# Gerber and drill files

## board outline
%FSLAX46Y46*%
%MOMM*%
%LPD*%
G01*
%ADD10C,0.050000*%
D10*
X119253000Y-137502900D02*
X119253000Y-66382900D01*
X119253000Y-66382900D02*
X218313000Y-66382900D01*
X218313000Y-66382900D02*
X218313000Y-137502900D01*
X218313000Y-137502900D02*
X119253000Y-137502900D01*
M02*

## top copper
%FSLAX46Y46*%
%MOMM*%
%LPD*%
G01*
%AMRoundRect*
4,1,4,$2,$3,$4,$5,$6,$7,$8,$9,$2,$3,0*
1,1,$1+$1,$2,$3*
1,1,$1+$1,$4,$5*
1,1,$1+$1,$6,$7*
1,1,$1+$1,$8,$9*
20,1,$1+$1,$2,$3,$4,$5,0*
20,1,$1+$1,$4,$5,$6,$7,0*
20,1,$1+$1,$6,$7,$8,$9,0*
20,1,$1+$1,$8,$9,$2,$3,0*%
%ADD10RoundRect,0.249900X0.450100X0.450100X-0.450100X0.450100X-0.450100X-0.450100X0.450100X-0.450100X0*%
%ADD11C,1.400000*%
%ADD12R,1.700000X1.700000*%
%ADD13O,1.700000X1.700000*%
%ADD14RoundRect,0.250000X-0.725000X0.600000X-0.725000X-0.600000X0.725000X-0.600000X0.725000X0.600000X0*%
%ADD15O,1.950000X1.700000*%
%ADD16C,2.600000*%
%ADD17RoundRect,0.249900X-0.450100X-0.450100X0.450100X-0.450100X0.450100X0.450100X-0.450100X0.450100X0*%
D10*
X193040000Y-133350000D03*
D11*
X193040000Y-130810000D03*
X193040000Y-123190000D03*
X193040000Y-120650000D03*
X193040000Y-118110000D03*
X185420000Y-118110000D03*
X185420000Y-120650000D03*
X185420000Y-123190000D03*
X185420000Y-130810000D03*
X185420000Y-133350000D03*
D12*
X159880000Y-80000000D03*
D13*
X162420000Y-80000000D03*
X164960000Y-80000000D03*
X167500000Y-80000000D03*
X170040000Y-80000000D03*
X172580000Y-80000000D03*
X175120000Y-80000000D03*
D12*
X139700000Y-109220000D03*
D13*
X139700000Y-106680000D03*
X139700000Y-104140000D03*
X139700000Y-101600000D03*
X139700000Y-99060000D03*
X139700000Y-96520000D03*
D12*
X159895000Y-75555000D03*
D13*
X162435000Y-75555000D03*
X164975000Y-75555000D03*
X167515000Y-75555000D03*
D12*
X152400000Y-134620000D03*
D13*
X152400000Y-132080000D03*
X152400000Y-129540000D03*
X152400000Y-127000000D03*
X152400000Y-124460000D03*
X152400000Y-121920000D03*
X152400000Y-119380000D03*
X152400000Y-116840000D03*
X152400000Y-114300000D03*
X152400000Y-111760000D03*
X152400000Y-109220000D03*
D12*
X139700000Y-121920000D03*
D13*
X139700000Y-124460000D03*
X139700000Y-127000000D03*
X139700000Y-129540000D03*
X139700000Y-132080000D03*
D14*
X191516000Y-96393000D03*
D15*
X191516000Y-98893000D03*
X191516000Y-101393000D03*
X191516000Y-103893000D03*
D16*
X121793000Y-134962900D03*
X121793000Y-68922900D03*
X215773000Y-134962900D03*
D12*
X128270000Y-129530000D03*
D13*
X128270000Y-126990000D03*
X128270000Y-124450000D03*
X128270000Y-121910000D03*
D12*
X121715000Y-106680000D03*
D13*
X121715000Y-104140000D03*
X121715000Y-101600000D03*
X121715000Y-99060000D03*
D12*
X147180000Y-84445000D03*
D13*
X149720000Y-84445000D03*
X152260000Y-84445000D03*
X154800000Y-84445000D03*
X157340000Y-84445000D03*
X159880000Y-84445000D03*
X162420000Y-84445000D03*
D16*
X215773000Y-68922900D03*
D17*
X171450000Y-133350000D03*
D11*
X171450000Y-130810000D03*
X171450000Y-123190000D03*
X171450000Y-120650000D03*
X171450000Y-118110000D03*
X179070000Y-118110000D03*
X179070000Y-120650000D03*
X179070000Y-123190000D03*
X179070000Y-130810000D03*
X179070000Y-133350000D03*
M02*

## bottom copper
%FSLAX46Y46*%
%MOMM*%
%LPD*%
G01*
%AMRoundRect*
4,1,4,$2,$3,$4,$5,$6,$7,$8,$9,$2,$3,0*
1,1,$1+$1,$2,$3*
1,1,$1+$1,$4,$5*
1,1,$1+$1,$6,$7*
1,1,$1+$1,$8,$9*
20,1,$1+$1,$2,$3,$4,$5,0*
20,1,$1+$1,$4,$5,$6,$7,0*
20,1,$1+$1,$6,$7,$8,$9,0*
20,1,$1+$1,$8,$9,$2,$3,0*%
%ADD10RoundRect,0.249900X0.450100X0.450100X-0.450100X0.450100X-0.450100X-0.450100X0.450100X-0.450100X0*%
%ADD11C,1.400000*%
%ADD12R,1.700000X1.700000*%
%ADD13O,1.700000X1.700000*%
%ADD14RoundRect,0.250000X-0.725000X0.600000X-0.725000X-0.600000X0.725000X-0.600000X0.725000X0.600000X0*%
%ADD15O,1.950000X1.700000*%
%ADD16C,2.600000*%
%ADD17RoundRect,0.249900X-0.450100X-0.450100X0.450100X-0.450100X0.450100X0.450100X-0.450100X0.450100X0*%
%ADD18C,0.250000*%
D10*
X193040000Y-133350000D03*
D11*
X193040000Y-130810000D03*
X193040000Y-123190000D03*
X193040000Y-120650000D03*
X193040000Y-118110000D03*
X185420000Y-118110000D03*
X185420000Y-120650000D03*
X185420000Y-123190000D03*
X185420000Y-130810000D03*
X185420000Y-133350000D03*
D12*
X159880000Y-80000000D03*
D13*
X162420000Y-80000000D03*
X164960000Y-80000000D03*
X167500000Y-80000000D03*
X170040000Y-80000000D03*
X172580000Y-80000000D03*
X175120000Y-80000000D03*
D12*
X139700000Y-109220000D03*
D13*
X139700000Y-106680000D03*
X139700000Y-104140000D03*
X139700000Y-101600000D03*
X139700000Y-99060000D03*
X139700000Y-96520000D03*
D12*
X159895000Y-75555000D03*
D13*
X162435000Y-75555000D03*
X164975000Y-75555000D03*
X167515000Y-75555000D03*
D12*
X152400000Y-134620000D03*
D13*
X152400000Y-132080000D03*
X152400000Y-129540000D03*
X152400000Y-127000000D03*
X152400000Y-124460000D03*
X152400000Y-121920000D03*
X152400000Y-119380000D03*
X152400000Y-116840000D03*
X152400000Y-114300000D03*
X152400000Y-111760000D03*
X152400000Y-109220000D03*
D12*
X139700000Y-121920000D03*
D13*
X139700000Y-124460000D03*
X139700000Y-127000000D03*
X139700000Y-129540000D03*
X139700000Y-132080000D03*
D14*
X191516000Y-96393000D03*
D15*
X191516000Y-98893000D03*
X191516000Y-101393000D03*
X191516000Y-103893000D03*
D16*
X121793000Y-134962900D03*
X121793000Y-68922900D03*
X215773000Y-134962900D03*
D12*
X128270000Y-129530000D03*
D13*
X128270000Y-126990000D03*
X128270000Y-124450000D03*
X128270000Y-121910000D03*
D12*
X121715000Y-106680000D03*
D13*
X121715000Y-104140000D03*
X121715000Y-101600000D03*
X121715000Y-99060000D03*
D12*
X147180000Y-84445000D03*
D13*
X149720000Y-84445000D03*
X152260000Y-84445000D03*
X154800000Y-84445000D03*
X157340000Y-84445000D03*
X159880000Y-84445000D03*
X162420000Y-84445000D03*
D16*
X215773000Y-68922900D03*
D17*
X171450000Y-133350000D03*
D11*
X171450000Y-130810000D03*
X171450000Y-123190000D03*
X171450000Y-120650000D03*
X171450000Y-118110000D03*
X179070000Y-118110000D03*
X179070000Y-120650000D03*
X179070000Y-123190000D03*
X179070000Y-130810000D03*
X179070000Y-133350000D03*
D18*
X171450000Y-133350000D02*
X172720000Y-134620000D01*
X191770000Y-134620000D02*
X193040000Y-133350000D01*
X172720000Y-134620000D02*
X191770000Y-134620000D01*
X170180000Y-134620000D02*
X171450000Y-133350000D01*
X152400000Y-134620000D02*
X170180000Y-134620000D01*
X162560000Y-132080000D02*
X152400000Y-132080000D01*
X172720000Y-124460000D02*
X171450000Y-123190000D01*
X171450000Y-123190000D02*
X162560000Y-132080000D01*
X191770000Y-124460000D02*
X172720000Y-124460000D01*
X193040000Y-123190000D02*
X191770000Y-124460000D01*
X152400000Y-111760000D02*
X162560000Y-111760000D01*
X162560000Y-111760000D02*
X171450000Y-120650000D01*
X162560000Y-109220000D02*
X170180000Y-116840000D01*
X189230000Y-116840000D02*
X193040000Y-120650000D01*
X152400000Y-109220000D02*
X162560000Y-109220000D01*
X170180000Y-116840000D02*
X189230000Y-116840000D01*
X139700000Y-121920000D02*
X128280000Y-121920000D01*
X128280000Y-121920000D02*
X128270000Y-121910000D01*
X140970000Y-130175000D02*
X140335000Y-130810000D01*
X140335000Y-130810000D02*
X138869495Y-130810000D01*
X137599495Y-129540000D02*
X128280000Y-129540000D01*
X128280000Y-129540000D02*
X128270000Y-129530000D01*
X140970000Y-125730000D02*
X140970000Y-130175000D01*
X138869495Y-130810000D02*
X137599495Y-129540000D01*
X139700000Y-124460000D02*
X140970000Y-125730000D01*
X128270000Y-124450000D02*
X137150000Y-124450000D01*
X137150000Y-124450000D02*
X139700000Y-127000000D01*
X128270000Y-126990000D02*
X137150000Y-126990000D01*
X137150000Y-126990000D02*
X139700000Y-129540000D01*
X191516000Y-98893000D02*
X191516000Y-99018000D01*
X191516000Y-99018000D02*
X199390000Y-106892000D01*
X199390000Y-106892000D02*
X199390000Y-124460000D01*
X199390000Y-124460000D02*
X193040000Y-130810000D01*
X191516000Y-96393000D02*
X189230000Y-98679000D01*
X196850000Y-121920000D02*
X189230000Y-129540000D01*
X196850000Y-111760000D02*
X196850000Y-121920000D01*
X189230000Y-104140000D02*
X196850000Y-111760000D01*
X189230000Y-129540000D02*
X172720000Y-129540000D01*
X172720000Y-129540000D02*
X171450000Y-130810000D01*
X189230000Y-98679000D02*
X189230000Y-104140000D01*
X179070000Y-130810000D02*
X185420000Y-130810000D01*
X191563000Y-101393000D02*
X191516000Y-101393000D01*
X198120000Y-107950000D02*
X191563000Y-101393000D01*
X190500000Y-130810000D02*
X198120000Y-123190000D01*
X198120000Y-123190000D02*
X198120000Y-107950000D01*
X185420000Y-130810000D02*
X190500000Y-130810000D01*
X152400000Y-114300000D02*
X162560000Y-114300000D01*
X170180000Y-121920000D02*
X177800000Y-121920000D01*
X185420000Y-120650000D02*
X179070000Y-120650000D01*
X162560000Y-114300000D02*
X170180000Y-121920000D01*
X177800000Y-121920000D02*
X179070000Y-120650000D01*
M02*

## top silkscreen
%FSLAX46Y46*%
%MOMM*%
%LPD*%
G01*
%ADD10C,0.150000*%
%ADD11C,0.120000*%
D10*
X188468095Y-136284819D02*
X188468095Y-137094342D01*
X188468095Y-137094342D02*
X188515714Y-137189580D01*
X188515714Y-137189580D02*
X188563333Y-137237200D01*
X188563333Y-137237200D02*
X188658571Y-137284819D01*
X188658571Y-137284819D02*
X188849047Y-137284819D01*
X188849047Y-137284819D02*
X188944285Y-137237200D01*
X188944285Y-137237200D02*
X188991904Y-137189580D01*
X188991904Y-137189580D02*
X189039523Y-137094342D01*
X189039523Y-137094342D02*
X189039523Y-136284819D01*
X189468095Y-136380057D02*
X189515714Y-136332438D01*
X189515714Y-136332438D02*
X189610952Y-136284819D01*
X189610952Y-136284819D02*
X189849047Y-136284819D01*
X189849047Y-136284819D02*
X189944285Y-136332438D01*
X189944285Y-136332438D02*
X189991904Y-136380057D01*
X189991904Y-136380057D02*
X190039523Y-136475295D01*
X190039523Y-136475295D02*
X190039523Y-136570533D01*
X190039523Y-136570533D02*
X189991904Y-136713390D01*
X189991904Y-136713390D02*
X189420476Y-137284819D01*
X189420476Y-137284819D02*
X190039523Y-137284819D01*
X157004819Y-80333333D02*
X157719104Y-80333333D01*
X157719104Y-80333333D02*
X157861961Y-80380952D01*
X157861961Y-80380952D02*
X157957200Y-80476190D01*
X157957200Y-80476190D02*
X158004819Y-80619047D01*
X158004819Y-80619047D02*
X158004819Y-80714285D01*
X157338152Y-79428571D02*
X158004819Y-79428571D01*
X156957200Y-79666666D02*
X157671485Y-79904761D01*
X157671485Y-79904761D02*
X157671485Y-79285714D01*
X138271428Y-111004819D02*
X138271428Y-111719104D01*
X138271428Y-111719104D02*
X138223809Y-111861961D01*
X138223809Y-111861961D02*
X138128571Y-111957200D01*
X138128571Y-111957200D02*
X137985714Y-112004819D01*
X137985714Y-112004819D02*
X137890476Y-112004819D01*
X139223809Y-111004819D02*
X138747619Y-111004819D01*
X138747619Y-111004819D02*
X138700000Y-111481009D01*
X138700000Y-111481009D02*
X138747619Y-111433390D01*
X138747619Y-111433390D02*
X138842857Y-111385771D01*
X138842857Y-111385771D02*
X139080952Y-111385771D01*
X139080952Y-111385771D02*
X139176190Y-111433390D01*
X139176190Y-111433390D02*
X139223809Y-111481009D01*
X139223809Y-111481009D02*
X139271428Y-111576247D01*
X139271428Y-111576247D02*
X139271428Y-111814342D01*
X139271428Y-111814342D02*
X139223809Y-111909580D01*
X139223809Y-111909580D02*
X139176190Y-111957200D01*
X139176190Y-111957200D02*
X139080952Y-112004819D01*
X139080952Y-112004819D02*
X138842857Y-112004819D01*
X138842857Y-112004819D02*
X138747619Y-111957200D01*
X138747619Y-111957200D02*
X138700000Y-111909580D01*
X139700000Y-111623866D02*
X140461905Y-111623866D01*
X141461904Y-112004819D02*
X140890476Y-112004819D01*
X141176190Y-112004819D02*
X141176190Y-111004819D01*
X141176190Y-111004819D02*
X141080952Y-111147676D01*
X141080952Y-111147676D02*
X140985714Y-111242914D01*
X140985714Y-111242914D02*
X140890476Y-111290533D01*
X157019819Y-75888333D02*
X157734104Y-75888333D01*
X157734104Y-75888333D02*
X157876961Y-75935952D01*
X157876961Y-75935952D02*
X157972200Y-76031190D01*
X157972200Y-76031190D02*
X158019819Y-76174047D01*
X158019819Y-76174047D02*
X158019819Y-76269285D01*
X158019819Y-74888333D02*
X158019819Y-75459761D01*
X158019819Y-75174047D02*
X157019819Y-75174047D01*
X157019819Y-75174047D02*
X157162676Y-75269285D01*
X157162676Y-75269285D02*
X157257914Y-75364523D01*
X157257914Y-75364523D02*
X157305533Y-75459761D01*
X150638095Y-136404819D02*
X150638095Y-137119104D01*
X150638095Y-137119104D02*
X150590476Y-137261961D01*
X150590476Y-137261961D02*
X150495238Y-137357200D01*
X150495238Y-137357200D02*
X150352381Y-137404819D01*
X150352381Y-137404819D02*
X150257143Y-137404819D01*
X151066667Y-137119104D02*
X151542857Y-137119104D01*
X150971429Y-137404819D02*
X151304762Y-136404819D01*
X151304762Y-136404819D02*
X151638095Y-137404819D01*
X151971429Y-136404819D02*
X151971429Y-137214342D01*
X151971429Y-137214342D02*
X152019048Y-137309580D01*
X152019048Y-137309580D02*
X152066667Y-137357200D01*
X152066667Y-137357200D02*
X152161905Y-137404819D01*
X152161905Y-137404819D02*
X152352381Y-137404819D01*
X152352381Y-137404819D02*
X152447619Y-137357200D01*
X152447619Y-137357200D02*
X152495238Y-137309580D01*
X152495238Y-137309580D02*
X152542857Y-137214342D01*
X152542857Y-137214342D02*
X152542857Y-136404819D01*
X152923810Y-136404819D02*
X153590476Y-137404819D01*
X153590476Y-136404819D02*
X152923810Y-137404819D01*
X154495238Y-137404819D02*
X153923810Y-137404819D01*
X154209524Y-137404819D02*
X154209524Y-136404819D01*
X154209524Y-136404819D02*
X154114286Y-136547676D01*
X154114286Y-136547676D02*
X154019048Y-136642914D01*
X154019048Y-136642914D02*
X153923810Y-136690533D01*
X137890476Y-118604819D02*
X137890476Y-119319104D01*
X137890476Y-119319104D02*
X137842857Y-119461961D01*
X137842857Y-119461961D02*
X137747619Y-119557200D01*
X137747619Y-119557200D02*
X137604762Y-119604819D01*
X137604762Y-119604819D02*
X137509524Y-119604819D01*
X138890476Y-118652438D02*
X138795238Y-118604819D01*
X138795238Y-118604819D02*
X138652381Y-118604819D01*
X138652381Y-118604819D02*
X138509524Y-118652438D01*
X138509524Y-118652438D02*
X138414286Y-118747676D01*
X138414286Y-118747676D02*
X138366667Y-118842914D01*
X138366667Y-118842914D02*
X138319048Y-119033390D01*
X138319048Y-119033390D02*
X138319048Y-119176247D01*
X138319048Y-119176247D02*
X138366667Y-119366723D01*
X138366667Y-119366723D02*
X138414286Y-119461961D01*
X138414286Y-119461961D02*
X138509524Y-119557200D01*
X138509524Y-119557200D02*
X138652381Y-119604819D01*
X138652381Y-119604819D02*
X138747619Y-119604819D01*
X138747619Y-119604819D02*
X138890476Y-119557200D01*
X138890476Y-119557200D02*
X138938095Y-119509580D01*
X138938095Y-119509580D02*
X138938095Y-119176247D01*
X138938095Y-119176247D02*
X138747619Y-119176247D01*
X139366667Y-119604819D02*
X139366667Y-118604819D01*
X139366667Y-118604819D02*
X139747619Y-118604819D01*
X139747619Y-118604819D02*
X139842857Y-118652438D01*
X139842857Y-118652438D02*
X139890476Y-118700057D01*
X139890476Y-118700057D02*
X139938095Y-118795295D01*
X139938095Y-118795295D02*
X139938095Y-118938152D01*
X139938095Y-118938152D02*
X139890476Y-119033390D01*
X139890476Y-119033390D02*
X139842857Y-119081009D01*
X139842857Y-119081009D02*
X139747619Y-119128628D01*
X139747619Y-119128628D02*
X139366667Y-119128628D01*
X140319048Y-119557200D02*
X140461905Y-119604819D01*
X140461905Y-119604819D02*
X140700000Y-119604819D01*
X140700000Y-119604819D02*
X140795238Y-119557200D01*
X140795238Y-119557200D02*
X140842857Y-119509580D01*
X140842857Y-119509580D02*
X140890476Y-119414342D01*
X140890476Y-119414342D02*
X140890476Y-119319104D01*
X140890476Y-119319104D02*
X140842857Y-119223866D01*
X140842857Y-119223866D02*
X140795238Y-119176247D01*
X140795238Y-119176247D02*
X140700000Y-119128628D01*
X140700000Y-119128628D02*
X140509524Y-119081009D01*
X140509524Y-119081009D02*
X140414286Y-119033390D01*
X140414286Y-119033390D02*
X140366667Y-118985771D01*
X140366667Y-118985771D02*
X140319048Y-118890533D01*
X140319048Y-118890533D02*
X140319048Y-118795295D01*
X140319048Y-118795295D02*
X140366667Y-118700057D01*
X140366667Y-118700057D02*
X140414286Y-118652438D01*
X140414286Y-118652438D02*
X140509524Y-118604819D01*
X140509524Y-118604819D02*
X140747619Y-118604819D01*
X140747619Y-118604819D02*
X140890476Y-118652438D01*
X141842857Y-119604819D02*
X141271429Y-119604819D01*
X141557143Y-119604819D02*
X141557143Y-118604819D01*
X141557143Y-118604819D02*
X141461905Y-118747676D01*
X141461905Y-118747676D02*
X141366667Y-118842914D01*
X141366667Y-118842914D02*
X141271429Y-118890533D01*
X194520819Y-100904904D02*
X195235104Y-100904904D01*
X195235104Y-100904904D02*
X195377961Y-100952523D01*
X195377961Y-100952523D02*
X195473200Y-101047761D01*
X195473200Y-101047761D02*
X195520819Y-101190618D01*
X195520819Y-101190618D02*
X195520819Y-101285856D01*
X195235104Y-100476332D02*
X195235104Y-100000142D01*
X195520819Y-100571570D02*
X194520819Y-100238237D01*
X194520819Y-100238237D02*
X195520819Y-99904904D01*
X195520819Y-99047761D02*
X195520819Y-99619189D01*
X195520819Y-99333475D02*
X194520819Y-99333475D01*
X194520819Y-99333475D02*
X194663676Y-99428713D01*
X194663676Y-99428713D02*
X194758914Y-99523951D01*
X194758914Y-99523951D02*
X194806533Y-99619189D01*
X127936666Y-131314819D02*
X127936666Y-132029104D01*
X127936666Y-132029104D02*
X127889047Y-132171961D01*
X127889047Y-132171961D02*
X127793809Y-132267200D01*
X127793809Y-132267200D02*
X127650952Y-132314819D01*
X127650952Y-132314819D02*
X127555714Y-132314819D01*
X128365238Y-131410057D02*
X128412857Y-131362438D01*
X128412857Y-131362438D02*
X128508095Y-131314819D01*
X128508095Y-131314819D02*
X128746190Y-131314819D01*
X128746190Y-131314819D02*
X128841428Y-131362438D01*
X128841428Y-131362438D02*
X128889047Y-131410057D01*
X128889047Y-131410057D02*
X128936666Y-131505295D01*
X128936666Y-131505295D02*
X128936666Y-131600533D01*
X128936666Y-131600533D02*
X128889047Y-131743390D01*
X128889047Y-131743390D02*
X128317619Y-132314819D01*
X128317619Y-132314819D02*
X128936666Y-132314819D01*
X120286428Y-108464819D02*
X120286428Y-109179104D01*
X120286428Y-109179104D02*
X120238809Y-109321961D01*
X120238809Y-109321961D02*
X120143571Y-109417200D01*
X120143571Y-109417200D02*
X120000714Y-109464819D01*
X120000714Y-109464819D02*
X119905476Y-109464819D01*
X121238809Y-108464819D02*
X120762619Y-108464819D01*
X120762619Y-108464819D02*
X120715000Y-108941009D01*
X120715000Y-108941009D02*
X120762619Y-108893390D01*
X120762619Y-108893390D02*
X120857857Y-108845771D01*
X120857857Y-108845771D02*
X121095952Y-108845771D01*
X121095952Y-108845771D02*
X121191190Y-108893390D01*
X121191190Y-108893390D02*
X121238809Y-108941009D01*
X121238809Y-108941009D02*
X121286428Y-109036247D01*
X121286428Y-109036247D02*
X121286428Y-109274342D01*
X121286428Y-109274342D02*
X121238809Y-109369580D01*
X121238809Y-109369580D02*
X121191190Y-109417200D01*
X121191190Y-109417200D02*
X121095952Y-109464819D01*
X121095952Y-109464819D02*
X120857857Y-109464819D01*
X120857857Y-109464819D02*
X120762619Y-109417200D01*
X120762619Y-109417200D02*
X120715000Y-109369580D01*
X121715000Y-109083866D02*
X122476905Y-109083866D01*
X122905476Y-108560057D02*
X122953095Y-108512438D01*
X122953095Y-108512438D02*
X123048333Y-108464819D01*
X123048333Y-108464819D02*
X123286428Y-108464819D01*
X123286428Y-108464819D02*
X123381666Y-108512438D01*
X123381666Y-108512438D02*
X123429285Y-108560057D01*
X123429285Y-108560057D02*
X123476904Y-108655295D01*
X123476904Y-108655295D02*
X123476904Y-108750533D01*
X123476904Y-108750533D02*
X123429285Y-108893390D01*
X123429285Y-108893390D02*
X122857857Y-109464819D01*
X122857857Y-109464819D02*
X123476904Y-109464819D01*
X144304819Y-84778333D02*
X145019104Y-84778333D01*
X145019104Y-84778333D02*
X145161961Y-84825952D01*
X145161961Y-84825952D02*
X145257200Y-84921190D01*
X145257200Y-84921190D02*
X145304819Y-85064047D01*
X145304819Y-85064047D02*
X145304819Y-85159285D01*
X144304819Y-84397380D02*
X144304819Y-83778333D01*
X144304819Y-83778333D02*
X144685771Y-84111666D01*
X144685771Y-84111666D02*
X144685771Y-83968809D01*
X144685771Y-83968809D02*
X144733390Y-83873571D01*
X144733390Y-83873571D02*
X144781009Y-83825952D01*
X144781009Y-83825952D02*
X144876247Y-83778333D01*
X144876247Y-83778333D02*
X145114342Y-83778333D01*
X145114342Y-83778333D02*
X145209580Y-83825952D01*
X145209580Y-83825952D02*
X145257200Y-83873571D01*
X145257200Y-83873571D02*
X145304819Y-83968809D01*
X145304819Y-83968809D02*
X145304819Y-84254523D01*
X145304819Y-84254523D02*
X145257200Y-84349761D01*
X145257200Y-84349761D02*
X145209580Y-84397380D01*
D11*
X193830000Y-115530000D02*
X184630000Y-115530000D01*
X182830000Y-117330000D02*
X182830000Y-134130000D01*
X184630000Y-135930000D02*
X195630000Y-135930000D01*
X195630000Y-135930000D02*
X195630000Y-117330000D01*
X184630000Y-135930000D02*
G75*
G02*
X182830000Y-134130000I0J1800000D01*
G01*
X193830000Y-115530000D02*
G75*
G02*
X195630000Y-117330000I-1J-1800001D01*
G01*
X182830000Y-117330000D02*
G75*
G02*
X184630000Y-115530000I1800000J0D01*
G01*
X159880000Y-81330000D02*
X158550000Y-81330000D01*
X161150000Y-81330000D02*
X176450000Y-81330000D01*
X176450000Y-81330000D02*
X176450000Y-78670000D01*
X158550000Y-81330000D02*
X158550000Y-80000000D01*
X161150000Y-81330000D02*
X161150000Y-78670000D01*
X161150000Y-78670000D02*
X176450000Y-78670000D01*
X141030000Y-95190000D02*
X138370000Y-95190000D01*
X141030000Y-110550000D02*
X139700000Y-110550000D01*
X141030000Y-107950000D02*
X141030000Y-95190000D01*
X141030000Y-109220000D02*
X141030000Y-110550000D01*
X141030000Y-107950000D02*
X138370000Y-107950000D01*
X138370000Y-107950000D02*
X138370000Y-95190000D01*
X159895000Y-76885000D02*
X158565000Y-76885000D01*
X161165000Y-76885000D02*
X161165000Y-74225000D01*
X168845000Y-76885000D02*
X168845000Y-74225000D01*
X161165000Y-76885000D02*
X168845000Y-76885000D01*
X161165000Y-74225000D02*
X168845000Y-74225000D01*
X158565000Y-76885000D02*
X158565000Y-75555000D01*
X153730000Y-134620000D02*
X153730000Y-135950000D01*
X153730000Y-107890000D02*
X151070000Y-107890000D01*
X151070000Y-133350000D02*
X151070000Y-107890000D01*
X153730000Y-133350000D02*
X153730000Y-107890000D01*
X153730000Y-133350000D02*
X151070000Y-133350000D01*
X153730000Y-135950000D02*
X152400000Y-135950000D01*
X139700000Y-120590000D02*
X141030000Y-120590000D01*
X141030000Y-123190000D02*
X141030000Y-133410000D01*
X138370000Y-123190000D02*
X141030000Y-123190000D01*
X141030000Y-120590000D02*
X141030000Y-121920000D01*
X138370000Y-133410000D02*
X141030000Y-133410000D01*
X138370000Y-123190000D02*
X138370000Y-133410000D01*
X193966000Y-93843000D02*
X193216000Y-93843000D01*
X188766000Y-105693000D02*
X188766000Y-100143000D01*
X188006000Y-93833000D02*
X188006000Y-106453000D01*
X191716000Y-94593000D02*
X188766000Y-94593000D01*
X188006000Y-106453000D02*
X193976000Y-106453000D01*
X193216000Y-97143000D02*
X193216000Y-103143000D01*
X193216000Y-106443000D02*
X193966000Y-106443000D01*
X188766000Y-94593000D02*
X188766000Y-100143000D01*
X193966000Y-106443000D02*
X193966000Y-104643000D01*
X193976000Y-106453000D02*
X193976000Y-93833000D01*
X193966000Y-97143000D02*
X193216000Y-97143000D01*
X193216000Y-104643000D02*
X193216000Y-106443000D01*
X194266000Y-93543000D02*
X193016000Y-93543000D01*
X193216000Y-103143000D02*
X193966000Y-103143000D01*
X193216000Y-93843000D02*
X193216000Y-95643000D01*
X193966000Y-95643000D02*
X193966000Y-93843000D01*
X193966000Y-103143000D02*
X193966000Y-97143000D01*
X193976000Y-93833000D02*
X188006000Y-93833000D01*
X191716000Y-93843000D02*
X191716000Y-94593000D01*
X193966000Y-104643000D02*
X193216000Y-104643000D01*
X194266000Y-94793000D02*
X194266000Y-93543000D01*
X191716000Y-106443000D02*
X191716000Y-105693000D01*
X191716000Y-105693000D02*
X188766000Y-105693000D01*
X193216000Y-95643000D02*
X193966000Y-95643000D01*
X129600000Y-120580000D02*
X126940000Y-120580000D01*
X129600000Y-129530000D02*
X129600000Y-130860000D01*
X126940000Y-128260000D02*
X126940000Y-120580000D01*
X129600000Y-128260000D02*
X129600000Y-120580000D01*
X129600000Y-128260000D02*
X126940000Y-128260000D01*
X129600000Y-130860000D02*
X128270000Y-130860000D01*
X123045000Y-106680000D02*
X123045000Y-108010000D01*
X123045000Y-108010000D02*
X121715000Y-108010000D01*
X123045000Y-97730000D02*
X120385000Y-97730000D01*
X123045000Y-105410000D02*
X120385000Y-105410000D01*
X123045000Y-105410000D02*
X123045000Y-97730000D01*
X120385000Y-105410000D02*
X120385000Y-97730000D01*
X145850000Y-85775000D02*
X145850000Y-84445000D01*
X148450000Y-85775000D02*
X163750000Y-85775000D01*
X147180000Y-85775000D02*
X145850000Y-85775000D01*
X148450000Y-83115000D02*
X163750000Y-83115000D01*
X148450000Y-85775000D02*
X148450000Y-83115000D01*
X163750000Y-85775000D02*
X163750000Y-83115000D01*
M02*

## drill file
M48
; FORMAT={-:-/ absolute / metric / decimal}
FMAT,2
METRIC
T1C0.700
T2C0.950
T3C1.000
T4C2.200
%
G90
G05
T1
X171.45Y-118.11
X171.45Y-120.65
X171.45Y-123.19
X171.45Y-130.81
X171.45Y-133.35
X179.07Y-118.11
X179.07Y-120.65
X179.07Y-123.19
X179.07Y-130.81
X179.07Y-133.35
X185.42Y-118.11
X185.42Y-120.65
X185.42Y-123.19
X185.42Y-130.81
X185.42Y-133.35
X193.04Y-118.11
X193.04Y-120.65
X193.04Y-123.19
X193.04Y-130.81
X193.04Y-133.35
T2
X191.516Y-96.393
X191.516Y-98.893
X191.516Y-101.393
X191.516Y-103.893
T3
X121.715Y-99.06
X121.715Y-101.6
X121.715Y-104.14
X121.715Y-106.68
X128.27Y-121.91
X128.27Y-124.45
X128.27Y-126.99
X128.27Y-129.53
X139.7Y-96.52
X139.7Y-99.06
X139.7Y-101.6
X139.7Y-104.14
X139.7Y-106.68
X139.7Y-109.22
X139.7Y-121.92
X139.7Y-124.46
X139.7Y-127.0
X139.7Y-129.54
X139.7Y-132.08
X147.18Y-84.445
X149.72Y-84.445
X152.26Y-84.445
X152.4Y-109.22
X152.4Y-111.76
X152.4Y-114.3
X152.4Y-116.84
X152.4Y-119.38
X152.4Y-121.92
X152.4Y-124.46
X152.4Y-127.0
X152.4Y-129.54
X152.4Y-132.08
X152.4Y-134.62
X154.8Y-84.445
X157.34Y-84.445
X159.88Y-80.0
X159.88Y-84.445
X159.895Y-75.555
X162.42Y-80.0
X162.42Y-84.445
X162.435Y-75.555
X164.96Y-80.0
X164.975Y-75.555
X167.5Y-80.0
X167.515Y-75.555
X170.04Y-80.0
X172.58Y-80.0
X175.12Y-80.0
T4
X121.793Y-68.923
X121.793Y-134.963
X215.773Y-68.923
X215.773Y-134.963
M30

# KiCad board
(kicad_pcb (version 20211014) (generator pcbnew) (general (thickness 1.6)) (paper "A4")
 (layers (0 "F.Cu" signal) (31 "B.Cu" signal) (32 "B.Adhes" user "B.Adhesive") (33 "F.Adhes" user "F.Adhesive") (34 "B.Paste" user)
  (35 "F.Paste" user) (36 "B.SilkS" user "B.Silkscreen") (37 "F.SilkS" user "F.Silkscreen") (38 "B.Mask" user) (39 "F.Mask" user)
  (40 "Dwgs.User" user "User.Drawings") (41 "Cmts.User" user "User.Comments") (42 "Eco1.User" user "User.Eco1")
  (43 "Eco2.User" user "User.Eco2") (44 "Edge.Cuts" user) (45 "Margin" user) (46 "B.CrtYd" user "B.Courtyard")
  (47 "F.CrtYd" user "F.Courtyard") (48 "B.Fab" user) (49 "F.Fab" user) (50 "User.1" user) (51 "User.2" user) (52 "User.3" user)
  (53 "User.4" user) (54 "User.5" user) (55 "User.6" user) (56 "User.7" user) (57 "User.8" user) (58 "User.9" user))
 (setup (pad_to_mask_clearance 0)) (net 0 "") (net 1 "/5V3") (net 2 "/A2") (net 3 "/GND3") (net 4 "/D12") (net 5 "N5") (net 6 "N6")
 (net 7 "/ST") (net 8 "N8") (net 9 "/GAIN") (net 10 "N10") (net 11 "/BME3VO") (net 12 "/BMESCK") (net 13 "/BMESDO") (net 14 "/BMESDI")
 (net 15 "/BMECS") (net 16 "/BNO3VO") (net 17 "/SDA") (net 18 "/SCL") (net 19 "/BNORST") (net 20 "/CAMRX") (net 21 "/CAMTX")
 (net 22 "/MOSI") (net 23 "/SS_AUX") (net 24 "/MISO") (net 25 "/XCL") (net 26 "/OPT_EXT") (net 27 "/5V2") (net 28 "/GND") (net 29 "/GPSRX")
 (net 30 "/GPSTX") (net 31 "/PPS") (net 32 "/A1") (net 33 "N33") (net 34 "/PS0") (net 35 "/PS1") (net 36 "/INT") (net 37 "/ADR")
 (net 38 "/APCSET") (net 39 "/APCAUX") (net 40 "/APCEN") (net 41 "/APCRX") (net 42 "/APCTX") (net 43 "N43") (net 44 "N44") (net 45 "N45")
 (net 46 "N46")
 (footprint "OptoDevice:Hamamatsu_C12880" (layer "F.Cu") (at 193.04 133.35 180)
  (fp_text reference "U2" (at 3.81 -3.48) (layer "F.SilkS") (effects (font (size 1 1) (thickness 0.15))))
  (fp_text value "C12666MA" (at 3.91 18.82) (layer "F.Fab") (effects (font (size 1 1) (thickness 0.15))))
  (fp_line (start -0.79 17.82) (end 8.41 17.82) (layer "F.SilkS") (width 0.12))
  (fp_line (start 10.21 16.02) (end 10.21 -0.78) (layer "F.SilkS") (width 0.12))
  (fp_line (start 8.41 -2.58) (end -2.59 -2.58) (layer "F.SilkS") (width 0.12))
  (fp_line (start -2.59 -2.58) (end -2.59 16.02) (layer "F.SilkS") (width 0.12))
  (fp_arc (start 8.41 -2.58) (mid 9.682792 -2.052792) (end 10.21 -0.78) (layer "F.SilkS") (width 0.12))
  (fp_arc (start -0.79 17.82) (mid -2.062792 17.292792) (end -2.59 16.02) (layer "F.SilkS") (width 0.12))
  (fp_arc (start 10.21 16.02) (mid 9.682792 17.292792) (end 8.41 17.82) (layer "F.SilkS") (width 0.12))
  (pad "1" thru_hole roundrect (at 0 0 180) (size 1.4 1.4) (drill 0.7) (layers *.Cu *.Mask) (roundrect_rratio 0.1785) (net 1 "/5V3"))
  (pad "2" thru_hole circle (at 0 2.54 180) (size 1.4 1.4) (drill 0.7) (layers *.Cu *.Mask) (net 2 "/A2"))
  (pad "3" thru_hole circle (at 0 10.16 180) (size 1.4 1.4) (drill 0.7) (layers *.Cu *.Mask) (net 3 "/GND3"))
  (pad "4" thru_hole circle (at 0 12.7 180) (size 1.4 1.4) (drill 0.7) (layers *.Cu *.Mask) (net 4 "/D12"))
  (pad "5" thru_hole circle (at 0 15.24 180) (size 1.4 1.4) (drill 0.7) (layers *.Cu *.Mask) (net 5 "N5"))
  (pad "6" thru_hole circle (at 7.62 15.24 180) (size 1.4 1.4) (drill 0.7) (layers *.Cu *.Mask) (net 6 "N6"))
  (pad "7" thru_hole circle (at 7.62 12.7 180) (size 1.4 1.4) (drill 0.7) (layers *.Cu *.Mask) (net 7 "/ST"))
  (pad "8" thru_hole circle (at 7.62 10.16 180) (size 1.4 1.4) (drill 0.7) (layers *.Cu *.Mask) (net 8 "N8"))
  (pad "9" thru_hole circle (at 7.62 2.54 180) (size 1.4 1.4) (drill 0.7) (layers *.Cu *.Mask) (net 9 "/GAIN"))
  (pad "10" thru_hole circle (at 7.62 0 180) (size 1.4 1.4) (drill 0.7) (layers *.Cu *.Mask) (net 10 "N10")))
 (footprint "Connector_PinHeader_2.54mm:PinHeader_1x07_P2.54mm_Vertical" (layer "F.Cu") (at 159.88 80 90)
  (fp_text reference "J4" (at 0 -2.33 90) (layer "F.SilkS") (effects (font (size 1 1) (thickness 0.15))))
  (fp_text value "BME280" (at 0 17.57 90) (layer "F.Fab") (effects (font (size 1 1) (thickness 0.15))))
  (fp_line (start -1.33 0) (end -1.33 -1.33) (layer "F.SilkS") (width 0.12))
  (fp_line (start -1.33 1.27) (end -1.33 16.57) (layer "F.SilkS") (width 0.12))
  (fp_line (start -1.33 16.57) (end 1.33 16.57) (layer "F.SilkS") (width 0.12))
  (fp_line (start -1.33 -1.33) (end 0 -1.33) (layer "F.SilkS") (width 0.12))
  (fp_line (start -1.33 1.27) (end 1.33 1.27) (layer "F.SilkS") (width 0.12))
  (fp_line (start 1.33 1.27) (end 1.33 16.57) (layer "F.SilkS") (width 0.12))
  (pad "1" thru_hole rect (at 0 0 90) (size 1.7 1.7) (drill 1) (layers *.Cu *.Mask) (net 1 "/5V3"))
  (pad "2" thru_hole oval (at 0 2.54 90) (size 1.7 1.7) (drill 1) (layers *.Cu *.Mask) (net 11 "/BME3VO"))
  (pad "3" thru_hole oval (at 0 5.08 90) (size 1.7 1.7) (drill 1) (layers *.Cu *.Mask) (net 3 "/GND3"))
  (pad "4" thru_hole oval (at 0 7.62 90) (size 1.7 1.7) (drill 1) (layers *.Cu *.Mask) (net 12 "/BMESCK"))
  (pad "5" thru_hole oval (at 0 10.16 90) (size 1.7 1.7) (drill 1) (layers *.Cu *.Mask) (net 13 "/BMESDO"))
  (pad "6" thru_hole oval (at 0 12.7 90) (size 1.7 1.7) (drill 1) (layers *.Cu *.Mask) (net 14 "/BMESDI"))
  (pad "7" thru_hole oval (at 0 15.24 90) (size 1.7 1.7) (drill 1) (layers *.Cu *.Mask) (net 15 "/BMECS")))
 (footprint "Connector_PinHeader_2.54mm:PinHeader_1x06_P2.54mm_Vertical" (layer "F.Cu") (at 139.7 109.22 180)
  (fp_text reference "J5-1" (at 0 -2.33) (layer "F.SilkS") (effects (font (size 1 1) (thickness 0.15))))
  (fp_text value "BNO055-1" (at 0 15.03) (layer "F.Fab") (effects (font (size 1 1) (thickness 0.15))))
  (fp_line (start -1.33 14.03) (end 1.33 14.03) (layer "F.SilkS") (width 0.12))
  (fp_line (start -1.33 -1.33) (end 0 -1.33) (layer "F.SilkS") (width 0.12))
  (fp_line (start -1.33 1.27) (end -1.33 14.03) (layer "F.SilkS") (width 0.12))
  (fp_line (start -1.33 0) (end -1.33 -1.33) (layer "F.SilkS") (width 0.12))
  (fp_line (start -1.33 1.27) (end 1.33 1.27) (layer "F.SilkS") (width 0.12))
  (fp_line (start 1.33 1.27) (end 1.33 14.03) (layer "F.SilkS") (width 0.12))
  (pad "1" thru_hole rect (at 0 0 180) (size 1.7 1.7) (drill 1) (layers *.Cu *.Mask) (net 1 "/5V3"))
  (pad "2" thru_hole oval (at 0 2.54 180) (size 1.7 1.7) (drill 1) (layers *.Cu *.Mask) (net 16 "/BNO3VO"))
  (pad "3" thru_hole oval (at 0 5.08 180) (size 1.7 1.7) (drill 1) (layers *.Cu *.Mask) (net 3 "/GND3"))
  (pad "4" thru_hole oval (at 0 7.62 180) (size 1.7 1.7) (drill 1) (layers *.Cu *.Mask) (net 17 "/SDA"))
  (pad "5" thru_hole oval (at 0 10.16 180) (size 1.7 1.7) (drill 1) (layers *.Cu *.Mask) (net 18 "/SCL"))
  (pad "6" thru_hole oval (at 0 12.7 180) (size 1.7 1.7) (drill 1) (layers *.Cu *.Mask) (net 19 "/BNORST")))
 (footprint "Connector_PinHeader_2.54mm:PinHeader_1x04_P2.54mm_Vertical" (layer "F.Cu") (at 159.895 75.555 90)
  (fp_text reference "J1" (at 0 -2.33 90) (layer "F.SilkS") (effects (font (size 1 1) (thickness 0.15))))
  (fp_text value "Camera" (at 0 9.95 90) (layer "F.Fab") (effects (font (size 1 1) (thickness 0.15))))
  (fp_line (start -1.33 0) (end -1.33 -1.33) (layer "F.SilkS") (width 0.12))
  (fp_line (start -1.33 1.27) (end 1.33 1.27) (layer "F.SilkS") (width 0.12))
  (fp_line (start -1.33 8.95) (end 1.33 8.95) (layer "F.SilkS") (width 0.12))
  (fp_line (start -1.33 1.27) (end -1.33 8.95) (layer "F.SilkS") (width 0.12))
  (fp_line (start 1.33 1.27) (end 1.33 8.95) (layer "F.SilkS") (width 0.12))
  (fp_line (start -1.33 -1.33) (end 0 -1.33) (layer "F.SilkS") (width 0.12))
  (pad "1" thru_hole rect (at 0 0 90) (size 1.7 1.7) (drill 1) (layers *.Cu *.Mask) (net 1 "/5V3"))
  (pad "2" thru_hole oval (at 0 2.54 90) (size 1.7 1.7) (drill 1) (layers *.Cu *.Mask) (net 3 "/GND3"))
  (pad "3" thru_hole oval (at 0 5.08 90) (size 1.7 1.7) (drill 1) (layers *.Cu *.Mask) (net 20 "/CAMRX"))
  (pad "4" thru_hole oval (at 0 7.62 90) (size 1.7 1.7) (drill 1) (layers *.Cu *.Mask) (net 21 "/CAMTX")))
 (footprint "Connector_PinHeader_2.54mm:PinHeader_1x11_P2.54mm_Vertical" (layer "F.Cu") (at 152.4 134.62 180)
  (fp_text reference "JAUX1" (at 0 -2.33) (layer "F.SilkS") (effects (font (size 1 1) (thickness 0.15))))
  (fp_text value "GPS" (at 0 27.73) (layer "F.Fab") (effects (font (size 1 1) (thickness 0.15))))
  (fp_line (start -1.33 0) (end -1.33 -1.33) (layer "F.SilkS") (width 0.12))
  (fp_line (start -1.33 26.73) (end 1.33 26.73) (layer "F.SilkS") (width 0.12))
  (fp_line (start 1.33 1.27) (end 1.33 26.73) (layer "F.SilkS") (width 0.12))
  (fp_line (start -1.33 1.27) (end -1.33 26.73) (layer "F.SilkS") (width 0.12))
  (fp_line (start -1.33 1.27) (end 1.33 1.27) (layer "F.SilkS") (width 0.12))
  (fp_line (start -1.33 -1.33) (end 0 -1.33) (layer "F.SilkS") (width 0.12))
  (pad "1" thru_hole rect (at 0 0 180) (size 1.7 1.7) (drill 1) (layers *.Cu *.Mask) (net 1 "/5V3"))
  (pad "2" thru_hole oval (at 0 2.54 180) (size 1.7 1.7) (drill 1) (layers *.Cu *.Mask) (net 3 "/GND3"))
  (pad "3" thru_hole oval (at 0 5.08 180) (size 1.7 1.7) (drill 1) (layers *.Cu *.Mask) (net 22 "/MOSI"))
  (pad "4" thru_hole oval (at 0 7.62 180) (size 1.7 1.7) (drill 1) (layers *.Cu *.Mask) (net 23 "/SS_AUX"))
  (pad "5" thru_hole oval (at 0 10.16 180) (size 1.7 1.7) (drill 1) (layers *.Cu *.Mask) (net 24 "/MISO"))
  (pad "6" thru_hole oval (at 0 12.7 180) (size 1.7 1.7) (drill 1) (layers *.Cu *.Mask) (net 18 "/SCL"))
  (pad "7" thru_hole oval (at 0 15.24 180) (size 1.7 1.7) (drill 1) (layers *.Cu *.Mask) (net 17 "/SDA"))
  (pad "8" thru_hole oval (at 0 17.78 180) (size 1.7 1.7) (drill 1) (layers *.Cu *.Mask) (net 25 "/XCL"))
  (pad "9" thru_hole oval (at 0 20.32 180) (size 1.7 1.7) (drill 1) (layers *.Cu *.Mask) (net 7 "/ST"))
  (pad "10" thru_hole oval (at 0 22.86 180) (size 1.7 1.7) (drill 1) (layers *.Cu *.Mask) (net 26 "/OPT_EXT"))
  (pad "11" thru_hole oval (at 0 25.4 180) (size 1.7 1.7) (drill 1) (layers *.Cu *.Mask) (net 4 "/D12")))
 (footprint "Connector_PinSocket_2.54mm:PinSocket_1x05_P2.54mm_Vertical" (layer "F.Cu") (at 139.7 121.92)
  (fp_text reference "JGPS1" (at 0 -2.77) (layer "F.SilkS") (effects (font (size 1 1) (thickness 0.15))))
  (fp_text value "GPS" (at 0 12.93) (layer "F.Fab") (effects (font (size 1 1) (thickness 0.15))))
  (fp_line (start 0 -1.33) (end 1.33 -1.33) (layer "F.SilkS") (width 0.12))
  (fp_line (start 1.33 1.27) (end 1.33 11.49) (layer "F.SilkS") (width 0.12))
  (fp_line (start -1.33 1.27) (end 1.33 1.27) (layer "F.SilkS") (width 0.12))
  (fp_line (start 1.33 -1.33) (end 1.33 0) (layer "F.SilkS") (width 0.12))
  (fp_line (start -1.33 11.49) (end 1.33 11.49) (layer "F.SilkS") (width 0.12))
  (fp_line (start -1.33 1.27) (end -1.33 11.49) (layer "F.SilkS") (width 0.12))
  (pad "1" thru_hole rect (at 0 0) (size 1.7 1.7) (drill 1) (layers *.Cu *.Mask) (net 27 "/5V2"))
  (pad "2" thru_hole oval (at 0 2.54) (size 1.7 1.7) (drill 1) (layers *.Cu *.Mask) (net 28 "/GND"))
  (pad "3" thru_hole oval (at 0 5.08) (size 1.7 1.7) (drill 1) (layers *.Cu *.Mask) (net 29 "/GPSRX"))
  (pad "4" thru_hole oval (at 0 7.62) (size 1.7 1.7) (drill 1) (layers *.Cu *.Mask) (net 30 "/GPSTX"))
  (pad "5" thru_hole oval (at 0 10.16) (size 1.7 1.7) (drill 1) (layers *.Cu *.Mask) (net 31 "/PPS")))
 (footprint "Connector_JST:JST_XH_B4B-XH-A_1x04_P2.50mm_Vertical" (layer "F.Cu") (at 191.516 96.393 -90)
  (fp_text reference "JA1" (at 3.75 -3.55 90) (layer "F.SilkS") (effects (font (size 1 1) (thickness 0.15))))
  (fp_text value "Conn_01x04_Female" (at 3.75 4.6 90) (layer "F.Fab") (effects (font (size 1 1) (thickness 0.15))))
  (fp_line (start -2.55 -2.45) (end -2.55 -1.7) (layer "F.SilkS") (width 0.12))
  (fp_line (start 9.3 2.75) (end 3.75 2.75) (layer "F.SilkS") (width 0.12))
  (fp_line (start -2.56 3.51) (end 10.06 3.51) (layer "F.SilkS") (width 0.12))
  (fp_line (start -1.8 -0.2) (end -1.8 2.75) (layer "F.SilkS") (width 0.12))
  (fp_line (start 10.06 3.51) (end 10.06 -2.46) (layer "F.SilkS") (width 0.12))
  (fp_line (start 0.75 -1.7) (end 6.75 -1.7) (layer "F.SilkS") (width 0.12))
  (fp_line (start 10.05 -1.7) (end 10.05 -2.45) (layer "F.SilkS") (width 0.12))
  (fp_line (start -1.8 2.75) (end 3.75 2.75) (layer "F.SilkS") (width 0.12))
  (fp_line (start 10.05 -2.45) (end 8.25 -2.45) (layer "F.SilkS") (width 0.12))
  (fp_line (start 10.06 -2.46) (end -2.56 -2.46) (layer "F.SilkS") (width 0.12))
  (fp_line (start 0.75 -2.45) (end 0.75 -1.7) (layer "F.SilkS") (width 0.12))
  (fp_line (start 8.25 -1.7) (end 10.05 -1.7) (layer "F.SilkS") (width 0.12))
  (fp_line (start -2.85 -2.75) (end -2.85 -1.5) (layer "F.SilkS") (width 0.12))
  (fp_line (start 6.75 -1.7) (end 6.75 -2.45) (layer "F.SilkS") (width 0.12))
  (fp_line (start -2.55 -1.7) (end -0.75 -1.7) (layer "F.SilkS") (width 0.12))
  (fp_line (start -0.75 -2.45) (end -2.55 -2.45) (layer "F.SilkS") (width 0.12))
  (fp_line (start 6.75 -2.45) (end 0.75 -2.45) (layer "F.SilkS") (width 0.12))
  (fp_line (start -2.56 -2.46) (end -2.56 3.51) (layer "F.SilkS") (width 0.12))
  (fp_line (start -2.55 -0.2) (end -1.8 -0.2) (layer "F.SilkS") (width 0.12))
  (fp_line (start 8.25 -2.45) (end 8.25 -1.7) (layer "F.SilkS") (width 0.12))
  (fp_line (start -1.6 -2.75) (end -2.85 -2.75) (layer "F.SilkS") (width 0.12))
  (fp_line (start 10.05 -0.2) (end 9.3 -0.2) (layer "F.SilkS") (width 0.12))
  (fp_line (start 9.3 -0.2) (end 9.3 2.75) (layer "F.SilkS") (width 0.12))
  (fp_line (start -0.75 -1.7) (end -0.75 -2.45) (layer "F.SilkS") (width 0.12))
  (pad "1" thru_hole roundrect (at 0 0 270) (size 1.7 1.95) (drill 0.95) (layers *.Cu *.Mask) (roundrect_rratio 0.147059) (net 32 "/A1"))
  (pad "2" thru_hole oval (at 2.5 0 270) (size 1.7 1.95) (drill 0.95) (layers *.Cu *.Mask) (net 2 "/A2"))
  (pad "3" thru_hole oval (at 5 0 270) (size 1.7 1.95) (drill 0.95) (layers *.Cu *.Mask) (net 9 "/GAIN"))
  (pad "4" thru_hole oval (at 7.5 0 270) (size 1.7 1.95) (drill 0.95) (layers *.Cu *.Mask) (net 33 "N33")))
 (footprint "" (layer "F.Cu") (at 121.793 134.9629)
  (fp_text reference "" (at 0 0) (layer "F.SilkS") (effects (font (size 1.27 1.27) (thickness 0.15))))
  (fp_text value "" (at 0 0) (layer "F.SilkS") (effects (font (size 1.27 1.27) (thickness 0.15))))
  (pad "1" thru_hole circle locked (at 0 0) (size 2.6 2.6) (drill 2.2) (layers *.Cu *.Mask)))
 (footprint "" (layer "F.Cu") (at 121.793 68.9229)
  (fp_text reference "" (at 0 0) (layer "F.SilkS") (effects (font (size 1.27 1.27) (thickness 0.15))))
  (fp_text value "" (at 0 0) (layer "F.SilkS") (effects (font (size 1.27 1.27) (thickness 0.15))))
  (pad "1" thru_hole circle locked (at 0 0) (size 2.6 2.6) (drill 2.2) (layers *.Cu *.Mask)))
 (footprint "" (layer "F.Cu") (at 215.773 134.9629)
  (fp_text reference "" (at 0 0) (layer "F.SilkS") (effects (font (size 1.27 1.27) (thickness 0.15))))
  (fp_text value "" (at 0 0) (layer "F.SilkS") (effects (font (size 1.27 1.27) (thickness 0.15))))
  (pad "1" thru_hole circle locked (at 0 0) (size 2.6 2.6) (drill 2.2) (layers *.Cu *.Mask)))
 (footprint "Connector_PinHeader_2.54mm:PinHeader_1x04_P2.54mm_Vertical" (layer "F.Cu") (at 128.27 129.53 180)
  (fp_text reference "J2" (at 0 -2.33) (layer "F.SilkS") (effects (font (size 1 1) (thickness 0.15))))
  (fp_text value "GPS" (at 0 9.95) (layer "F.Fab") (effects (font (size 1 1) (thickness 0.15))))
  (fp_line (start -1.33 8.95) (end 1.33 8.95) (layer "F.SilkS") (width 0.12))
  (fp_line (start -1.33 0) (end -1.33 -1.33) (layer "F.SilkS") (width 0.12))
  (fp_line (start 1.33 1.27) (end 1.33 8.95) (layer "F.SilkS") (width 0.12))
  (fp_line (start -1.33 1.27) (end -1.33 8.95) (layer "F.SilkS") (width 0.12))
  (fp_line (start -1.33 1.27) (end 1.33 1.27) (layer "F.SilkS") (width 0.12))
  (fp_line (start -1.33 -1.33) (end 0 -1.33) (layer "F.SilkS") (width 0.12))
  (pad "1" thru_hole rect (at 0 0 180) (size 1.7 1.7) (drill 1) (layers *.Cu *.Mask) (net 28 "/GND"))
  (pad "2" thru_hole oval (at 0 2.54 180) (size 1.7 1.7) (drill 1) (layers *.Cu *.Mask) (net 30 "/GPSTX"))
  (pad "3" thru_hole oval (at 0 5.08 180) (size 1.7 1.7) (drill 1) (layers *.Cu *.Mask) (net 29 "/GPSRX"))
  (pad "4" thru_hole oval (at 0 7.62 180) (size 1.7 1.7) (drill 1) (layers *.Cu *.Mask) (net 27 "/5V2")))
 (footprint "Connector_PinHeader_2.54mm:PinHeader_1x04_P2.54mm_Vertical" (layer "F.Cu") (at 121.715 106.68 180)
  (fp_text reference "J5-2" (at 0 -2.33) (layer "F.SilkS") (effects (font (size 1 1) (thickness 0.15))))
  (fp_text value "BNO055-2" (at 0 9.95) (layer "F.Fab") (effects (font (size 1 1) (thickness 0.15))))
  (fp_line (start -1.33 0) (end -1.33 -1.33) (layer "F.SilkS") (width 0.12))
  (fp_line (start -1.33 -1.33) (end 0 -1.33) (layer "F.SilkS") (width 0.12))
  (fp_line (start -1.33 8.95) (end 1.33 8.95) (layer "F.SilkS") (width 0.12))
  (fp_line (start -1.33 1.27) (end 1.33 1.27) (layer "F.SilkS") (width 0.12))
  (fp_line (start -1.33 1.27) (end -1.33 8.95) (layer "F.SilkS") (width 0.12))
  (fp_line (start 1.33 1.27) (end 1.33 8.95) (layer "F.SilkS") (width 0.12))
  (pad "1" thru_hole rect (at 0 0 180) (size 1.7 1.7) (drill 1) (layers *.Cu *.Mask) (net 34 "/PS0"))
  (pad "2" thru_hole oval (at 0 2.54 180) (size 1.7 1.7) (drill 1) (layers *.Cu *.Mask) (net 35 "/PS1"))
  (pad "3" thru_hole oval (at 0 5.08 180) (size 1.7 1.7) (drill 1) (layers *.Cu *.Mask) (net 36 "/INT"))
  (pad "4" thru_hole oval (at 0 7.62 180) (size 1.7 1.7) (drill 1) (layers *.Cu *.Mask) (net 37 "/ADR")))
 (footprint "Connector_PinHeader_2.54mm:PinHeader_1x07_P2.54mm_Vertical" (layer "F.Cu") (at 147.18 84.445 90)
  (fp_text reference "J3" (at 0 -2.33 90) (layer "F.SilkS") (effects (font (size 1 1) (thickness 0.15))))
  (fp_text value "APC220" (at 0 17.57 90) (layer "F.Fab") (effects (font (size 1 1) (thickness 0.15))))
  (fp_line (start -1.33 -1.33) (end 0 -1.33) (layer "F.SilkS") (width 0.12))
  (fp_line (start -1.33 1.27) (end -1.33 16.57) (layer "F.SilkS") (width 0.12))
  (fp_line (start -1.33 0) (end -1.33 -1.33) (layer "F.SilkS") (width 0.12))
  (fp_line (start 1.33 1.27) (end 1.33 16.57) (layer "F.SilkS") (width 0.12))
  (fp_line (start -1.33 1.27) (end 1.33 1.27) (layer "F.SilkS") (width 0.12))
  (fp_line (start -1.33 16.57) (end 1.33 16.57) (layer "F.SilkS") (width 0.12))
  (pad "1" thru_hole rect (at 0 0 90) (size 1.7 1.7) (drill 1) (layers *.Cu *.Mask) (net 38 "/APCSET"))
  (pad "2" thru_hole oval (at 0 2.54 90) (size 1.7 1.7) (drill 1) (layers *.Cu *.Mask) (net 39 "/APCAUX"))
  (pad "3" thru_hole oval (at 0 5.08 90) (size 1.7 1.7) (drill 1) (layers *.Cu *.Mask) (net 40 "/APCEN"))
  (pad "4" thru_hole oval (at 0 7.62 90) (size 1.7 1.7) (drill 1) (layers *.Cu *.Mask) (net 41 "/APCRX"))
  (pad "5" thru_hole oval (at 0 10.16 90) (size 1.7 1.7) (drill 1) (layers *.Cu *.Mask) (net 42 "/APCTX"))
  (pad "6" thru_hole oval (at 0 12.7 90) (size 1.7 1.7) (drill 1) (layers *.Cu *.Mask) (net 1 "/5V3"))
  (pad "7" thru_hole oval (at 0 15.24 90) (size 1.7 1.7) (drill 1) (layers *.Cu *.Mask) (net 3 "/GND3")))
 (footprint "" (layer "F.Cu") (at 215.773 68.9229)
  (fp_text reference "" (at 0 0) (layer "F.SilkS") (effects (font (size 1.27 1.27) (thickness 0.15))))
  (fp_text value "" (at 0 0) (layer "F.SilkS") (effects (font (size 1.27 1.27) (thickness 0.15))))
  (pad "1" thru_hole circle locked (at 0 0) (size 2.6 2.6) (drill 2.2) (layers *.Cu *.Mask)))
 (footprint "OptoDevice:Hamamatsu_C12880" (layer "B.Cu") (at 171.45 133.35)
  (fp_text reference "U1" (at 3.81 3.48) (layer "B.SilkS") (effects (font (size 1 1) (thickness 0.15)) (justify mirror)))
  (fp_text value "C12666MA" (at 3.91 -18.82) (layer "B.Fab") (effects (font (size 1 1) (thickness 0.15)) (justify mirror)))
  (pad "1" thru_hole roundrect (at 0 0) (size 1.4 1.4) (drill 0.7) (layers *.Cu *.Mask) (roundrect_rratio 0.1785) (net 1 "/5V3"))
  (pad "2" thru_hole circle (at 0 -2.54) (size 1.4 1.4) (drill 0.7) (layers *.Cu *.Mask) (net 32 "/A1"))
  (pad "3" thru_hole circle (at 0 -10.16) (size 1.4 1.4) (drill 0.7) (layers *.Cu *.Mask) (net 3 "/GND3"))
  (pad "4" thru_hole circle (at 0 -12.7) (size 1.4 1.4) (drill 0.7) (layers *.Cu *.Mask) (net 26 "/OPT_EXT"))
  (pad "5" thru_hole circle (at 0 -15.24) (size 1.4 1.4) (drill 0.7) (layers *.Cu *.Mask) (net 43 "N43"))
  (pad "6" thru_hole circle (at 7.62 -15.24) (size 1.4 1.4) (drill 0.7) (layers *.Cu *.Mask) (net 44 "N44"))
  (pad "7" thru_hole circle (at 7.62 -12.7) (size 1.4 1.4) (drill 0.7) (layers *.Cu *.Mask) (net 7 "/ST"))
  (pad "8" thru_hole circle (at 7.62 -10.16) (size 1.4 1.4) (drill 0.7) (layers *.Cu *.Mask) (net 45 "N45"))
  (pad "9" thru_hole circle (at 7.62 -2.54) (size 1.4 1.4) (drill 0.7) (layers *.Cu *.Mask) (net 9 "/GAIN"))
  (pad "10" thru_hole circle (at 7.62 0) (size 1.4 1.4) (drill 0.7) (layers *.Cu *.Mask) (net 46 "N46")))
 (gr_line (start 119.253 137.5029) (end 119.253 66.3829) (layer "Edge.Cuts") (width 0.05))
 (gr_line (start 119.253 66.3829) (end 218.313 66.3829) (layer "Edge.Cuts") (width 0.05))
 (gr_line (start 218.313 66.3829) (end 218.313 137.5029) (layer "Edge.Cuts") (width 0.05))
 (gr_line (start 218.313 137.5029) (end 119.253 137.5029) (layer "Edge.Cuts") (width 0.05))
 (segment (start 171.45 133.35) (end 172.72 134.62) (width 0.25) (layer "B.Cu") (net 1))
 (segment (start 191.77 134.62) (end 193.04 133.35) (width 0.25) (layer "B.Cu") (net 1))
 (segment (start 172.72 134.62) (end 191.77 134.62) (width 0.25) (layer "B.Cu") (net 1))
 (segment (start 170.18 134.62) (end 171.45 133.35) (width 0.25) (layer "B.Cu") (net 1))
 (segment (start 152.4 134.62) (end 170.18 134.62) (width 0.25) (layer "B.Cu") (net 1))
 (segment (start 162.56 132.08) (end 152.4 132.08) (width 0.25) (layer "B.Cu") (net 3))
 (segment (start 172.72 124.46) (end 171.45 123.19) (width 0.25) (layer "B.Cu") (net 3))
 (segment (start 171.45 123.19) (end 162.56 132.08) (width 0.25) (layer "B.Cu") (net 3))
 (segment (start 191.77 124.46) (end 172.72 124.46) (width 0.25) (layer "B.Cu") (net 3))
 (segment (start 193.04 123.19) (end 191.77 124.46) (width 0.25) (layer "B.Cu") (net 3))
 (segment (start 152.4 111.76) (end 162.56 111.76) (width 0.25) (layer "B.Cu") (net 26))
 (segment (start 162.56 111.76) (end 171.45 120.65) (width 0.25) (layer "B.Cu") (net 26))
 (segment (start 162.56 109.22) (end 170.18 116.84) (width 0.25) (layer "B.Cu") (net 4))
 (segment (start 189.23 116.84) (end 193.04 120.65) (width 0.25) (layer "B.Cu") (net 4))
 (segment (start 152.4 109.22) (end 162.56 109.22) (width 0.25) (layer "B.Cu") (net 4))
 (segment (start 170.18 116.84) (end 189.23 116.84) (width 0.25) (layer "B.Cu") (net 4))
 (segment (start 139.7 121.92) (end 128.28 121.92) (width 0.25) (layer "B.Cu") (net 27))
 (segment (start 128.28 121.92) (end 128.27 121.91) (width 0.25) (layer "B.Cu") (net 27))
 (segment (start 140.97 130.175) (end 140.335 130.81) (width 0.25) (layer "B.Cu") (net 28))
 (segment (start 140.335 130.81) (end 138.869495 130.81) (width 0.25) (layer "B.Cu") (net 28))
 (segment locked (start 137.599495 129.54) (end 128.28 129.54) (width 0.25) (layer "B.Cu") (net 28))
 (segment (start 128.28 129.54) (end 128.27 129.53) (width 0.25) (layer "B.Cu") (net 28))
 (segment (start 140.97 125.73) (end 140.97 130.175) (width 0.25) (layer "B.Cu") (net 28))
 (segment (start 138.869495 130.81) (end 137.599495 129.54) (width 0.25) (layer "B.Cu") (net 28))
 (segment (start 139.7 124.46) (end 140.97 125.73) (width 0.25) (layer "B.Cu") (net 28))
 (segment (start 128.27 124.45) (end 137.15 124.45) (width 0.25) (layer "B.Cu") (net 29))
 (segment (start 137.15 124.45) (end 139.7 127) (width 0.25) (layer "B.Cu") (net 29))
 (segment (start 128.27 126.99) (end 137.15 126.99) (width 0.25) (layer "B.Cu") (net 30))
 (segment (start 137.15 126.99) (end 139.7 129.54) (width 0.25) (layer "B.Cu") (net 30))
 (segment (start 191.516 98.893) (end 191.516 99.018) (width 0.25) (layer "B.Cu") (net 2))
 (segment (start 191.516 99.018) (end 199.39 106.892) (width 0.25) (layer "B.Cu") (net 2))
 (segment (start 199.39 106.892) (end 199.39 124.46) (width 0.25) (layer "B.Cu") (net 2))
 (segment (start 199.39 124.46) (end 193.04 130.81) (width 0.25) (layer "B.Cu") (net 2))
 (segment (start 191.516 96.393) (end 189.23 98.679) (width 0.25) (layer "B.Cu") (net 32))
 (segment (start 196.85 121.92) (end 189.23 129.54) (width 0.25) (layer "B.Cu") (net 32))
 (segment (start 196.85 111.76) (end 196.85 121.92) (width 0.25) (layer "B.Cu") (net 32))
 (segment (start 189.23 104.14) (end 196.85 111.76) (width 0.25) (layer "B.Cu") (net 32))
 (segment (start 189.23 129.54) (end 172.72 129.54) (width 0.25) (layer "B.Cu") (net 32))
 (segment (start 172.72 129.54) (end 171.45 130.81) (width 0.25) (layer "B.Cu") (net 32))
 (segment (start 189.23 98.679) (end 189.23 104.14) (width 0.25) (layer "B.Cu") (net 32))
 (segment (start 179.07 130.81) (end 185.42 130.81) (width 0.25) (layer "B.Cu") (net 9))
 (segment (start 191.563 101.393) (end 191.516 101.393) (width 0.25) (layer "B.Cu") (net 9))
 (segment (start 198.12 107.95) (end 191.563 101.393) (width 0.25) (layer "B.Cu") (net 9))
 (segment (start 190.5 130.81) (end 198.12 123.19) (width 0.25) (layer "B.Cu") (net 9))
 (segment (start 198.12 123.19) (end 198.12 107.95) (width 0.25) (layer "B.Cu") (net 9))
 (segment (start 185.42 130.81) (end 190.5 130.81) (width 0.25) (layer "B.Cu") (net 9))
 (segment (start 152.4 114.3) (end 162.56 114.3) (width 0.25) (layer "B.Cu") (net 7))
 (segment (start 170.18 121.92) (end 177.8 121.92) (width 0.25) (layer "B.Cu") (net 7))
 (segment (start 185.42 120.65) (end 179.07 120.65) (width 0.25) (layer "B.Cu") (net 7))
 (segment (start 162.56 114.3) (end 170.18 121.92) (width 0.25) (layer "B.Cu") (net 7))
 (segment (start 177.8 121.92) (end 179.07 120.65) (width 0.25) (layer "B.Cu") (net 7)))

